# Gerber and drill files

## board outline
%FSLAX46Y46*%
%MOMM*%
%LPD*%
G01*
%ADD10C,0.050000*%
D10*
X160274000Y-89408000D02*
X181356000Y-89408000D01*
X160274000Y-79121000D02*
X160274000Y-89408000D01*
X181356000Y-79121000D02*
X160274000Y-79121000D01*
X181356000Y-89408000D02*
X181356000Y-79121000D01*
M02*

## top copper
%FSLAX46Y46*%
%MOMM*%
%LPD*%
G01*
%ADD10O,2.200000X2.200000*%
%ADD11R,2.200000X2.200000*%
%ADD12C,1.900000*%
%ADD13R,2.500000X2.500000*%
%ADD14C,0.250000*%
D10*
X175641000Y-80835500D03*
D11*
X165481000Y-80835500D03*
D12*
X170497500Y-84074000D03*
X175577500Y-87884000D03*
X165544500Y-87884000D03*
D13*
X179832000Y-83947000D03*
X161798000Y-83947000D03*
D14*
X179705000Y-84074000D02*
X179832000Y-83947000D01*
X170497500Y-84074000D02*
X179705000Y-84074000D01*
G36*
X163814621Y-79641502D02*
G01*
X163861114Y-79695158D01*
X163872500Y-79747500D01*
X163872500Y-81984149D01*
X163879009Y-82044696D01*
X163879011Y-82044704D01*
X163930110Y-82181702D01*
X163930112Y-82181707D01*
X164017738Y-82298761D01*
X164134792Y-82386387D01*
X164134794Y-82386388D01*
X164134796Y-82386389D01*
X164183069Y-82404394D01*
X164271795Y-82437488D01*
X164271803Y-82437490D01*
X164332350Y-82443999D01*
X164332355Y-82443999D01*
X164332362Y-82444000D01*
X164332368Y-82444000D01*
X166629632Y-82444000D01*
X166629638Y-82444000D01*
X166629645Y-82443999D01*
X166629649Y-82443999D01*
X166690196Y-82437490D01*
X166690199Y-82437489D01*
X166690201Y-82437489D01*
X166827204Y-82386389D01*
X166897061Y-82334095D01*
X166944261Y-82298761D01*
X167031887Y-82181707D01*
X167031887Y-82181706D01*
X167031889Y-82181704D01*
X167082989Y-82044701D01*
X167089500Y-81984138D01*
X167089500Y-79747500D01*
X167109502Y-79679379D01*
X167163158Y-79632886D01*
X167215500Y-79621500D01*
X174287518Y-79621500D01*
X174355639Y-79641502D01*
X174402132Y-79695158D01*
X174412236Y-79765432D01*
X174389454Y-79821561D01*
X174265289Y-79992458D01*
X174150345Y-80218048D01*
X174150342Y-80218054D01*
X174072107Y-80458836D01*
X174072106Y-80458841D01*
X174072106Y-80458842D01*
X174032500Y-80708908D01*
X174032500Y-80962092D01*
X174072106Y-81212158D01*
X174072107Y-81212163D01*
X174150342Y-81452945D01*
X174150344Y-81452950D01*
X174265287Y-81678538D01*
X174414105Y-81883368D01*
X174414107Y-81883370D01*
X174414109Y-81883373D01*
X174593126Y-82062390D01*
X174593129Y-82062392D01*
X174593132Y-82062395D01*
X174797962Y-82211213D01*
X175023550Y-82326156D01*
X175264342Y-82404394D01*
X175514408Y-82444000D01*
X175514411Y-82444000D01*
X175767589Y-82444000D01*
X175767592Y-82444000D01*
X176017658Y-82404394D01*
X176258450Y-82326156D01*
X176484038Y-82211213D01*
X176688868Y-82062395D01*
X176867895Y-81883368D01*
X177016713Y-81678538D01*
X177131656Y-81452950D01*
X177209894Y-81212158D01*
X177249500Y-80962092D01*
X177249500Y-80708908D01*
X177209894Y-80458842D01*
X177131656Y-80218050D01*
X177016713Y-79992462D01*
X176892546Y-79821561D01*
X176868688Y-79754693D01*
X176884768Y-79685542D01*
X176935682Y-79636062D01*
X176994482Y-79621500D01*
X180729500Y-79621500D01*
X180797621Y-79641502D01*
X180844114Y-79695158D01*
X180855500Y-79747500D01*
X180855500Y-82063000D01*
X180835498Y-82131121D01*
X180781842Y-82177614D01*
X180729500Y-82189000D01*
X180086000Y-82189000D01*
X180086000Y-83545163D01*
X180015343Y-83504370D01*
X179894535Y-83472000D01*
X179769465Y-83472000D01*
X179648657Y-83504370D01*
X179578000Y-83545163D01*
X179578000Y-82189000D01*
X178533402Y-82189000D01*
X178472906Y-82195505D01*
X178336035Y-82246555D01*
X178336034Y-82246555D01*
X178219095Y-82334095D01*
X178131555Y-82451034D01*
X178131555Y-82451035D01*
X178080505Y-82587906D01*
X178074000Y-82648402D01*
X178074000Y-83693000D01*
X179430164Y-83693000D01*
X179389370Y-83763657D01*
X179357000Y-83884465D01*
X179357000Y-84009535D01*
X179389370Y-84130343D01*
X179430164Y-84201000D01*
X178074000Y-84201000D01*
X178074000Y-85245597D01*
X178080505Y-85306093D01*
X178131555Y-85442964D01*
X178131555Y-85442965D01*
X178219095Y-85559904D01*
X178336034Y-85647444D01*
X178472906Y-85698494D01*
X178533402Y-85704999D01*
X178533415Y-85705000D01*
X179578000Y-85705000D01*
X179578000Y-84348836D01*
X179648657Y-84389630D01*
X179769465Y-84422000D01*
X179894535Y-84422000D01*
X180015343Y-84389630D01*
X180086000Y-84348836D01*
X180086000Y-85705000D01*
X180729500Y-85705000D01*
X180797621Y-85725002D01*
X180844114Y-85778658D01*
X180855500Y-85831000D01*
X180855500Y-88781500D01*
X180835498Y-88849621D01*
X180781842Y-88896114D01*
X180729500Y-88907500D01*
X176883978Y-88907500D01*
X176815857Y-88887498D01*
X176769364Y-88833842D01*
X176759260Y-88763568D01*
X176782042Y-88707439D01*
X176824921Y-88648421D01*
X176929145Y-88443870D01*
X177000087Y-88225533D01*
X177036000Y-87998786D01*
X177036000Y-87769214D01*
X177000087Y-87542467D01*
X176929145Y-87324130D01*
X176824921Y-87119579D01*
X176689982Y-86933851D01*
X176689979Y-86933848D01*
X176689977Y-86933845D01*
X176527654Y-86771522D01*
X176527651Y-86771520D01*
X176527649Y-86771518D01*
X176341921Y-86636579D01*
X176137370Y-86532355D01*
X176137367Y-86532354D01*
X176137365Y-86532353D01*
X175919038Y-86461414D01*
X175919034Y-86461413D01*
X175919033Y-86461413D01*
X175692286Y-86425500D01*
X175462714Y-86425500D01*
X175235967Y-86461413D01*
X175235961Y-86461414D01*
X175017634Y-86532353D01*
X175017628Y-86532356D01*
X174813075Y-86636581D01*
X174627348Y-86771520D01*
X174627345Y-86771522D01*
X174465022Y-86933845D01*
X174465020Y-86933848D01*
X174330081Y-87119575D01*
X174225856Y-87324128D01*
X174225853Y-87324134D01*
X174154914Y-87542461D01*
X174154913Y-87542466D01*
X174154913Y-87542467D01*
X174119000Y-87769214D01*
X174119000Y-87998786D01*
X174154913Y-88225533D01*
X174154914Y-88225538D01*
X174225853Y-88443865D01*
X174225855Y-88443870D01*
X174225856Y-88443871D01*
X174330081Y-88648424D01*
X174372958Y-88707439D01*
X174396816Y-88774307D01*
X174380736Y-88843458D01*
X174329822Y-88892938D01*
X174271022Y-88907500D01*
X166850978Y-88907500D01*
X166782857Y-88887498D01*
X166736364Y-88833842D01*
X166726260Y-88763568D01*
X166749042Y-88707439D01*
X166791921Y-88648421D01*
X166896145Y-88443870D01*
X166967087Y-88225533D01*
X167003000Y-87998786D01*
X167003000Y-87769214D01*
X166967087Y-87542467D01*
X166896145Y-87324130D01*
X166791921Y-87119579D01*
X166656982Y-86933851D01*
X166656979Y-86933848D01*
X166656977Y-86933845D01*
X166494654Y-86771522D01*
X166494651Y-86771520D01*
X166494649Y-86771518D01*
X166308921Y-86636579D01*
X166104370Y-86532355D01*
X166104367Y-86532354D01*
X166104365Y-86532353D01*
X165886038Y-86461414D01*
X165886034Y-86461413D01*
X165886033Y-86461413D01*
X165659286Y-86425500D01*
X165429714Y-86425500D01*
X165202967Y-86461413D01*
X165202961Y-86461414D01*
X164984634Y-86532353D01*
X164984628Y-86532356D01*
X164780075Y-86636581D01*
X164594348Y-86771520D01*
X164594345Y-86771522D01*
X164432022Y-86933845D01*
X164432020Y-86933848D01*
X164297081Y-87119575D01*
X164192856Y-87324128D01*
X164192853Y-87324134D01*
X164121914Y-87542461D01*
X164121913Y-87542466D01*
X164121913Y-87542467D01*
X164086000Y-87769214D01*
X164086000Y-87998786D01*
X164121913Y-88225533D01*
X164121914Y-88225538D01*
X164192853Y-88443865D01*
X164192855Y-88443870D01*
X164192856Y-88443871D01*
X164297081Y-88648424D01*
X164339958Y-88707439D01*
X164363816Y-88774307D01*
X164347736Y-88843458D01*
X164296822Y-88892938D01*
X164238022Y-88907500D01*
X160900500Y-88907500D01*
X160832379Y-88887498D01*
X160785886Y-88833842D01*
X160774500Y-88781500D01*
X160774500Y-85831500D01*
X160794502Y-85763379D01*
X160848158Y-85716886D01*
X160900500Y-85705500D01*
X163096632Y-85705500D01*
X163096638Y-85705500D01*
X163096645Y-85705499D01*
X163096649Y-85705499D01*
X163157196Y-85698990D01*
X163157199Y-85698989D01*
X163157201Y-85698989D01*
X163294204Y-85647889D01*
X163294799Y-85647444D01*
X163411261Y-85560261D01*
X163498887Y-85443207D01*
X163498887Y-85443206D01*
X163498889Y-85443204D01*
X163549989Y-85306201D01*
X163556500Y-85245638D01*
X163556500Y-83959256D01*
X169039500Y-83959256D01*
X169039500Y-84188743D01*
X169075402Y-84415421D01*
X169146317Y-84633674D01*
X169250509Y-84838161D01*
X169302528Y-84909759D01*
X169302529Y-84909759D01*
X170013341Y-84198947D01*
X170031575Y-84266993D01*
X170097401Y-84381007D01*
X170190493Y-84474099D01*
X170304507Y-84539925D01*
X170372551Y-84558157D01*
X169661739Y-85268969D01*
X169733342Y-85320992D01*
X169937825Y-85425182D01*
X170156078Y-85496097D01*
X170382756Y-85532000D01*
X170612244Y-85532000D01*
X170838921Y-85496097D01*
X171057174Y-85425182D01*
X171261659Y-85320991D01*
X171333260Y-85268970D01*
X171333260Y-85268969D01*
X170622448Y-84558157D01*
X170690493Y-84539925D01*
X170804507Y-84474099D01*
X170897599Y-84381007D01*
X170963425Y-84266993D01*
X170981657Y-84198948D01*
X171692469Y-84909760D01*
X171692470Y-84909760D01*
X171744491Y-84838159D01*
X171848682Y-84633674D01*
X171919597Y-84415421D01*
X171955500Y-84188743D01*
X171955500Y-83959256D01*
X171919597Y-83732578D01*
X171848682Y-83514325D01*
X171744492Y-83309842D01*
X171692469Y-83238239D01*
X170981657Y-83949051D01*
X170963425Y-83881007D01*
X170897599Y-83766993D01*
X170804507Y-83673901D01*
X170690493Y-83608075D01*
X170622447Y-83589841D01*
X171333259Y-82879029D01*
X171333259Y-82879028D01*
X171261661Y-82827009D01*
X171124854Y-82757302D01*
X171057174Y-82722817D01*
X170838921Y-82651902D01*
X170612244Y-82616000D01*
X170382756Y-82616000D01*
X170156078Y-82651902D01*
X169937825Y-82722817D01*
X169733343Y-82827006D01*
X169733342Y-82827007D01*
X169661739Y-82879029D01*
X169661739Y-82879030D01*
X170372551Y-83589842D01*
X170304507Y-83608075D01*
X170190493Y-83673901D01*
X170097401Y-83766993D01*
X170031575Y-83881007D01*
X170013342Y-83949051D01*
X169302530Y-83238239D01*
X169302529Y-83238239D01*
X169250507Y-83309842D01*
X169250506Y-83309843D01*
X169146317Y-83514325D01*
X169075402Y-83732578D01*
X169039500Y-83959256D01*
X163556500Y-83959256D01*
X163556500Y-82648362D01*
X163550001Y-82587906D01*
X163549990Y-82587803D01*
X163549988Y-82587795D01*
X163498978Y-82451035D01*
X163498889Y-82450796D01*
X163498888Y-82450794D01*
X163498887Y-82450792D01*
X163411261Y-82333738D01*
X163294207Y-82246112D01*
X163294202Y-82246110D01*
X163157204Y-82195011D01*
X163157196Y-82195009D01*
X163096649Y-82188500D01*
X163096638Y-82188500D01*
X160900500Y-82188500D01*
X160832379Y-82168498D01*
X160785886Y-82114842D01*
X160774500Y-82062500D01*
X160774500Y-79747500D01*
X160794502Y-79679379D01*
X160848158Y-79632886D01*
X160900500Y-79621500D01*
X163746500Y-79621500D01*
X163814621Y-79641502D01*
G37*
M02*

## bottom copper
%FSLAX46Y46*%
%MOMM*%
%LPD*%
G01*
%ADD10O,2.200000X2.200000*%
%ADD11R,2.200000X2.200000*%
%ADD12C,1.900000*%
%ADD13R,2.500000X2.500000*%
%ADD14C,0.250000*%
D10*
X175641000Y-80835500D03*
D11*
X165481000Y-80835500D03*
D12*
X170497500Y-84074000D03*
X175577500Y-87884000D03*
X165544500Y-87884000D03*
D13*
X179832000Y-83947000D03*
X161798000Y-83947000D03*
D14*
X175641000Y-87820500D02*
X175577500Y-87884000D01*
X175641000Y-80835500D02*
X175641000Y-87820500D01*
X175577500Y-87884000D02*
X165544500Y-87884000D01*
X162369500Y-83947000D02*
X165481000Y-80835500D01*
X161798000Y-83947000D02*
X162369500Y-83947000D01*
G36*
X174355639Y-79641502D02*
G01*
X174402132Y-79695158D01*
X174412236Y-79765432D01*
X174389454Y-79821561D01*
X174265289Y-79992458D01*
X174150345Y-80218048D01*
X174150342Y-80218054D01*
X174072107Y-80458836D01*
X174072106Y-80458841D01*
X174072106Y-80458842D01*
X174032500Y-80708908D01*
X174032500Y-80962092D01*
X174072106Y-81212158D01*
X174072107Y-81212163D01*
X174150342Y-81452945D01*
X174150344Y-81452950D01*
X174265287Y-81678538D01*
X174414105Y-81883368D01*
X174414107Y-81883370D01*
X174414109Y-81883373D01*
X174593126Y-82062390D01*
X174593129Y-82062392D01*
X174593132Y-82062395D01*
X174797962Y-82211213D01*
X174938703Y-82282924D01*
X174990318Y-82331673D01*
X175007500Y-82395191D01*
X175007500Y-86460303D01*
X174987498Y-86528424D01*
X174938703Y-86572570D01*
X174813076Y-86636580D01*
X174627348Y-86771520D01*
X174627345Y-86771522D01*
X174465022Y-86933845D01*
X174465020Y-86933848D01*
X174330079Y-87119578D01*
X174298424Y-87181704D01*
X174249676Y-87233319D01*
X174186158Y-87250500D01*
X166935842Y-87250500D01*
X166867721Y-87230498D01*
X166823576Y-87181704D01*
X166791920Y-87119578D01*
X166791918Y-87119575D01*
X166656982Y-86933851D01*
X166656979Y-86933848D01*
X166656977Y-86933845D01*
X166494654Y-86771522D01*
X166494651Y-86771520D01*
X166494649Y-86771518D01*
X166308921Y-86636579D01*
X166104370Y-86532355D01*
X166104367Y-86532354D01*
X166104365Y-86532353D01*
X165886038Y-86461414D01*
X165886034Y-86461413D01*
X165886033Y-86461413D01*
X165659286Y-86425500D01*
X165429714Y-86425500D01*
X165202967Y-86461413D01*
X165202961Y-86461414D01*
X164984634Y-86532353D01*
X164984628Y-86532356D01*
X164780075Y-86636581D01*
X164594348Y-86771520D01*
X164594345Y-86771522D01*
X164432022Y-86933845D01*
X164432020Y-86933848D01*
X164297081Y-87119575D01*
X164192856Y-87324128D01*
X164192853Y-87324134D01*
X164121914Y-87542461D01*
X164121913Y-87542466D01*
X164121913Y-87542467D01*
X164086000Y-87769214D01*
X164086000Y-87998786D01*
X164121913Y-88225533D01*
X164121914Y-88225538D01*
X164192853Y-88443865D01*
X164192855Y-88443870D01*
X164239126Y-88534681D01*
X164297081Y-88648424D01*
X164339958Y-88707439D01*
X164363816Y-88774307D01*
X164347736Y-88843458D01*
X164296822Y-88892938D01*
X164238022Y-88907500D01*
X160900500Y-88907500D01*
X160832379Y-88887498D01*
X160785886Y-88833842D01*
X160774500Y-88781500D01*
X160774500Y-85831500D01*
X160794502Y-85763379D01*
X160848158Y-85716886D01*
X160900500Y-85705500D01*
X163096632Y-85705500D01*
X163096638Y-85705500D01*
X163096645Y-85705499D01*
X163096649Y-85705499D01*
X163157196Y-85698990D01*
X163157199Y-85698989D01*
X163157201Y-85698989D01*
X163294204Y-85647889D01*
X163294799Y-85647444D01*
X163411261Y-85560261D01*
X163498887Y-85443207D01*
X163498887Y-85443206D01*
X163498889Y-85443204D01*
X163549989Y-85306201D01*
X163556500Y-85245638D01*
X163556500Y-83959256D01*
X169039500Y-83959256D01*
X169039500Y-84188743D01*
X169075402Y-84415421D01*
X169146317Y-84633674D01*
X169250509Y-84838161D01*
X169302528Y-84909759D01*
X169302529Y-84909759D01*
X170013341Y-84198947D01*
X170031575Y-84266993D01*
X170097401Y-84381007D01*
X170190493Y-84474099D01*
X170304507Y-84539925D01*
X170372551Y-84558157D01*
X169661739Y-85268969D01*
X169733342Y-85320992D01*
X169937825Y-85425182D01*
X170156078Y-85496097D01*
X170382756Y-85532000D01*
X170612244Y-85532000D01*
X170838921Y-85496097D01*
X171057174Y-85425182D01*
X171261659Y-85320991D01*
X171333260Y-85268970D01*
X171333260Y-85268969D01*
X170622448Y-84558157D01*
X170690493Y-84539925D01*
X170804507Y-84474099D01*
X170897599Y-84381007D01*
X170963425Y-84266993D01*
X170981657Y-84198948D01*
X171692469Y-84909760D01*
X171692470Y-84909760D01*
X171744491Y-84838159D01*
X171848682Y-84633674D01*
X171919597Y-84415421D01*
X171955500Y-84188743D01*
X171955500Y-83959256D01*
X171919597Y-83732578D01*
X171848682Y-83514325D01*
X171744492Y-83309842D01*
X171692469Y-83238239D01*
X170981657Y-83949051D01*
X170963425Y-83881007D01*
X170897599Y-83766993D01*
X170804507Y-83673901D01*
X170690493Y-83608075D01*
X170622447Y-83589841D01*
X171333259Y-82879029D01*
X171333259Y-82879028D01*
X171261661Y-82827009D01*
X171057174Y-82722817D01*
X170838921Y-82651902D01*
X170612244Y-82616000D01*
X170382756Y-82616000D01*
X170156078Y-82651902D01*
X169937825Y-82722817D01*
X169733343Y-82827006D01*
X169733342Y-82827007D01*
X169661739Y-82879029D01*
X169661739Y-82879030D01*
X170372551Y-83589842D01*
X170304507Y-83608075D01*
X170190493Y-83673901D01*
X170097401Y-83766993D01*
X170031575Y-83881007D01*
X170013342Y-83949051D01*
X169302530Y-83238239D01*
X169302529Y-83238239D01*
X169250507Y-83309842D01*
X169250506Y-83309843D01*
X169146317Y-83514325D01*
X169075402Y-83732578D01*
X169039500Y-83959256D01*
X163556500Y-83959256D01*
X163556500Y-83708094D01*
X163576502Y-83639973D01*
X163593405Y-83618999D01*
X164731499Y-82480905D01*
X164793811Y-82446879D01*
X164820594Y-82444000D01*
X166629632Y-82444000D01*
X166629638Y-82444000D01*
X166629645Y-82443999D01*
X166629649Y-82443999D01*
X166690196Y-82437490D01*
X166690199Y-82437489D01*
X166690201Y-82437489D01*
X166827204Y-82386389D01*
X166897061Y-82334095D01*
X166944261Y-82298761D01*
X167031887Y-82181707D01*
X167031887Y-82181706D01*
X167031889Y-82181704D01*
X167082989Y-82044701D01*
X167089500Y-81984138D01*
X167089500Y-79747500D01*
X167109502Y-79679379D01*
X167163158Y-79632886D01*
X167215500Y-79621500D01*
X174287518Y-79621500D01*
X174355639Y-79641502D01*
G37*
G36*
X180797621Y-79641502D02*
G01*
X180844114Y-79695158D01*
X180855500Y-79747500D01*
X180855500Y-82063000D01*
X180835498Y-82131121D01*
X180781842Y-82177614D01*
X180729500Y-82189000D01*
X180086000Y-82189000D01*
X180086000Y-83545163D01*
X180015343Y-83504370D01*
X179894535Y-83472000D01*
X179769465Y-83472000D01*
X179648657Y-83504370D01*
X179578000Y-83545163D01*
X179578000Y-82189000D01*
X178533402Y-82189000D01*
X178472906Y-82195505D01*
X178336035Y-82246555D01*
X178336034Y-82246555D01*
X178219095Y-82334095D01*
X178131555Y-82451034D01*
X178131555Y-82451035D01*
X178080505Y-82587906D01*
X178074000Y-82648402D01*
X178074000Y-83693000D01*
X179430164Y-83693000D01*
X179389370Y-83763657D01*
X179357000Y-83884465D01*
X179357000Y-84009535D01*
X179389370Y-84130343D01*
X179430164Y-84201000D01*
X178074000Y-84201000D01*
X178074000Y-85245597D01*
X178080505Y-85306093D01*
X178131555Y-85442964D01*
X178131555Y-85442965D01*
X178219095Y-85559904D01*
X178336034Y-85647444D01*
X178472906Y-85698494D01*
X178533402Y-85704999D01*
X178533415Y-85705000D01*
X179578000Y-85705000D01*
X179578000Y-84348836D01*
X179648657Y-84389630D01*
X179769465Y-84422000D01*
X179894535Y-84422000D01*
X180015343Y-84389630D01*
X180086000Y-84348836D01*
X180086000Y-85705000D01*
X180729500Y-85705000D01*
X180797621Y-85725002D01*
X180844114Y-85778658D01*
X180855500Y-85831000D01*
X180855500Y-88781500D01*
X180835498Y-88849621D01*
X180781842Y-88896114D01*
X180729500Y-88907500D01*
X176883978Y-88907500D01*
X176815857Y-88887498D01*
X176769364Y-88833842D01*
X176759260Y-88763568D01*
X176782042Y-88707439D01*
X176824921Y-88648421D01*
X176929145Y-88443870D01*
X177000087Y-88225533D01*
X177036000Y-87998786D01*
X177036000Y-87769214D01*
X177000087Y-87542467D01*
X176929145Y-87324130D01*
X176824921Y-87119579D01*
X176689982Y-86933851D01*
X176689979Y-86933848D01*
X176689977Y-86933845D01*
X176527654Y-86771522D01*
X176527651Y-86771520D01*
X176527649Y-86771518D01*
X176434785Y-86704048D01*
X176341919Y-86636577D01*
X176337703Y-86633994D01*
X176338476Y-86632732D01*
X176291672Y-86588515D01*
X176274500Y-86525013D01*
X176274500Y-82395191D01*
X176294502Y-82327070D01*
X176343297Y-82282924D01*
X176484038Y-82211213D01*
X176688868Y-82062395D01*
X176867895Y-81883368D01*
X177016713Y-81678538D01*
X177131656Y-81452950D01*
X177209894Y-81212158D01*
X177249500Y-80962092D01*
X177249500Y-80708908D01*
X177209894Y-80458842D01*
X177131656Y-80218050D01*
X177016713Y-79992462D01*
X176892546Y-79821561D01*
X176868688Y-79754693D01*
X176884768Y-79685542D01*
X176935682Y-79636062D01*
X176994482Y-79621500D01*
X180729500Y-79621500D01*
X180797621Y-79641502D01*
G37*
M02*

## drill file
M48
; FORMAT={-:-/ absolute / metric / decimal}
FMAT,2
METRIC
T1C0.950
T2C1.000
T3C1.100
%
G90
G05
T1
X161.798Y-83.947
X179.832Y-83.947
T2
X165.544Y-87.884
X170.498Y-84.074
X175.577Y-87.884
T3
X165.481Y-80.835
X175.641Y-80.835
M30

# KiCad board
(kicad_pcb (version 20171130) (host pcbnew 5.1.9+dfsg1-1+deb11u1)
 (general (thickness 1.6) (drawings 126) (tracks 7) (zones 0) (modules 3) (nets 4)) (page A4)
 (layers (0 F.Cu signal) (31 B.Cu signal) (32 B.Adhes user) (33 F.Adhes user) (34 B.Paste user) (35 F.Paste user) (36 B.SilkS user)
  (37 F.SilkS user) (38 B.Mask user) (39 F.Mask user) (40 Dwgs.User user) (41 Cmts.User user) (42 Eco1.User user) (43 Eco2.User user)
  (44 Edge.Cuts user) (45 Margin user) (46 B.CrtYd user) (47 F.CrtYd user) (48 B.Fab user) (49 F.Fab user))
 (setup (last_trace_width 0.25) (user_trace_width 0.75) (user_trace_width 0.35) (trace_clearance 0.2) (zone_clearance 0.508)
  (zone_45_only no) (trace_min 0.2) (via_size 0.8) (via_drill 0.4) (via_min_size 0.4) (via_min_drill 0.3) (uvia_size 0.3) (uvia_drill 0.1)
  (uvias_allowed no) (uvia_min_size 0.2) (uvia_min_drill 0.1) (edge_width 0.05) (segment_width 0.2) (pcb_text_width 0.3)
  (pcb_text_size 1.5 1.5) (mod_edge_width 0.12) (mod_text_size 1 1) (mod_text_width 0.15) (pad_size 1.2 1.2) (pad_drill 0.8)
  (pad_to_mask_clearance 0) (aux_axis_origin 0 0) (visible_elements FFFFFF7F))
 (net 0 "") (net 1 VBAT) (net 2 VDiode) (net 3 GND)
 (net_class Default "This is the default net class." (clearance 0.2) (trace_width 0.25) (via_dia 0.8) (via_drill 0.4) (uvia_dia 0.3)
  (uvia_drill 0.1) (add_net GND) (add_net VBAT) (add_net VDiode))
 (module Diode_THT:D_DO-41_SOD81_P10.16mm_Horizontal (layer F.Cu) (at 165.481 80.8355)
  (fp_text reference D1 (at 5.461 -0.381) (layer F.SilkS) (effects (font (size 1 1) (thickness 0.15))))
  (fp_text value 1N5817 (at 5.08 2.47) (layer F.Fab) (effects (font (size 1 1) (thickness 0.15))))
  (pad 2 thru_hole oval (at 10.16 0) (size 2.2 2.2) (drill 1.1) (layers *.Cu *.Mask) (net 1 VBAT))
  (pad 1 thru_hole rect (at 0 0) (size 2.2 2.2) (drill 1.1) (layers *.Cu *.Mask) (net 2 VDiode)))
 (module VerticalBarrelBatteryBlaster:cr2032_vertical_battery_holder (layer F.Cu) (at 165.5445 87.884)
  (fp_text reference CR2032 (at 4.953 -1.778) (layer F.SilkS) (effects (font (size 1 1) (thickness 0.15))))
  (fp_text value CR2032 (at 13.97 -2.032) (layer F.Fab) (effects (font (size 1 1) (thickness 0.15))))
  (pad 2 thru_hole circle (at 4.953 -3.81) (size 1.9 1.9) (drill 1) (layers *.Cu *.Mask) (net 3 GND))
  (pad 1 thru_hole circle (at 10.033 0) (size 1.9 1.9) (drill 1) (layers *.Cu *.Mask) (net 1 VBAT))
  (pad 1 thru_hole circle (at 0 0) (size 1.9 1.9) (drill 1) (layers *.Cu *.Mask) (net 1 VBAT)))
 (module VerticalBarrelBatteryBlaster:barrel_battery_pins (layer B.Cu) (at 179.832 83.947 180)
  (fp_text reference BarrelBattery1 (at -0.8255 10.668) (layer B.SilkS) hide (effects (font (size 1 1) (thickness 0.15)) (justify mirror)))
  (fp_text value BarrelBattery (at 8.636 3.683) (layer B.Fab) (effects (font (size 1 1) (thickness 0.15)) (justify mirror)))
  (pad 2 thru_hole rect (at 0 0 90) (size 2.5 2.5) (drill 0.95) (layers *.Cu *.Mask) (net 3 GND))
  (pad 1 thru_hole rect (at 18.034 0 180) (size 2.5 2.5) (drill 0.95) (layers *.Cu *.Mask) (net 2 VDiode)))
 (gr_line (start 160.274 89.408) (end 181.356 89.408) (layer Edge.Cuts) (width 0.05))
 (gr_line (start 160.274 79.121) (end 160.274 89.408) (layer Edge.Cuts) (width 0.05))
 (gr_line (start 181.356 79.121) (end 160.274 79.121) (layer Edge.Cuts) (width 0.05))
 (gr_line (start 181.356 89.408) (end 181.356 79.121) (layer Edge.Cuts) (width 0.05))
 (segment (start 179.705 84.074) (end 179.832 83.947) (width 0.25) (layer F.Cu) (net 3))
 (segment (start 170.4975 84.074) (end 179.705 84.074) (width 0.25) (layer F.Cu) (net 3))
 (segment (start 175.641 87.8205) (end 175.5775 87.884) (width 0.25) (layer B.Cu) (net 1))
 (segment (start 175.641 80.8355) (end 175.641 87.8205) (width 0.25) (layer B.Cu) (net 1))
 (segment (start 175.5775 87.884) (end 165.5445 87.884) (width 0.25) (layer B.Cu) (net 1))
 (segment (start 162.3695 83.947) (end 165.481 80.8355) (width 0.25) (layer B.Cu) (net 2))
 (segment (start 161.798 83.947) (end 162.3695 83.947) (width 0.25) (layer B.Cu) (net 2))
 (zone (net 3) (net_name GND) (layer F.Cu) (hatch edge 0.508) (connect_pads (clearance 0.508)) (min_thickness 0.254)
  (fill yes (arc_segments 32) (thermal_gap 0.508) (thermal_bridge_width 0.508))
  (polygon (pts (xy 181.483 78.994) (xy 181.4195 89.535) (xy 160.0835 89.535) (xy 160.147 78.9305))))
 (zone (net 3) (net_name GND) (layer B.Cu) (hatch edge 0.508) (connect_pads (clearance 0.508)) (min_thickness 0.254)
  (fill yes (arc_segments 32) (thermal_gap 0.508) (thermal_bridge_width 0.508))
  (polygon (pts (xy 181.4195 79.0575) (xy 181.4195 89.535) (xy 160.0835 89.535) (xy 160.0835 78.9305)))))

